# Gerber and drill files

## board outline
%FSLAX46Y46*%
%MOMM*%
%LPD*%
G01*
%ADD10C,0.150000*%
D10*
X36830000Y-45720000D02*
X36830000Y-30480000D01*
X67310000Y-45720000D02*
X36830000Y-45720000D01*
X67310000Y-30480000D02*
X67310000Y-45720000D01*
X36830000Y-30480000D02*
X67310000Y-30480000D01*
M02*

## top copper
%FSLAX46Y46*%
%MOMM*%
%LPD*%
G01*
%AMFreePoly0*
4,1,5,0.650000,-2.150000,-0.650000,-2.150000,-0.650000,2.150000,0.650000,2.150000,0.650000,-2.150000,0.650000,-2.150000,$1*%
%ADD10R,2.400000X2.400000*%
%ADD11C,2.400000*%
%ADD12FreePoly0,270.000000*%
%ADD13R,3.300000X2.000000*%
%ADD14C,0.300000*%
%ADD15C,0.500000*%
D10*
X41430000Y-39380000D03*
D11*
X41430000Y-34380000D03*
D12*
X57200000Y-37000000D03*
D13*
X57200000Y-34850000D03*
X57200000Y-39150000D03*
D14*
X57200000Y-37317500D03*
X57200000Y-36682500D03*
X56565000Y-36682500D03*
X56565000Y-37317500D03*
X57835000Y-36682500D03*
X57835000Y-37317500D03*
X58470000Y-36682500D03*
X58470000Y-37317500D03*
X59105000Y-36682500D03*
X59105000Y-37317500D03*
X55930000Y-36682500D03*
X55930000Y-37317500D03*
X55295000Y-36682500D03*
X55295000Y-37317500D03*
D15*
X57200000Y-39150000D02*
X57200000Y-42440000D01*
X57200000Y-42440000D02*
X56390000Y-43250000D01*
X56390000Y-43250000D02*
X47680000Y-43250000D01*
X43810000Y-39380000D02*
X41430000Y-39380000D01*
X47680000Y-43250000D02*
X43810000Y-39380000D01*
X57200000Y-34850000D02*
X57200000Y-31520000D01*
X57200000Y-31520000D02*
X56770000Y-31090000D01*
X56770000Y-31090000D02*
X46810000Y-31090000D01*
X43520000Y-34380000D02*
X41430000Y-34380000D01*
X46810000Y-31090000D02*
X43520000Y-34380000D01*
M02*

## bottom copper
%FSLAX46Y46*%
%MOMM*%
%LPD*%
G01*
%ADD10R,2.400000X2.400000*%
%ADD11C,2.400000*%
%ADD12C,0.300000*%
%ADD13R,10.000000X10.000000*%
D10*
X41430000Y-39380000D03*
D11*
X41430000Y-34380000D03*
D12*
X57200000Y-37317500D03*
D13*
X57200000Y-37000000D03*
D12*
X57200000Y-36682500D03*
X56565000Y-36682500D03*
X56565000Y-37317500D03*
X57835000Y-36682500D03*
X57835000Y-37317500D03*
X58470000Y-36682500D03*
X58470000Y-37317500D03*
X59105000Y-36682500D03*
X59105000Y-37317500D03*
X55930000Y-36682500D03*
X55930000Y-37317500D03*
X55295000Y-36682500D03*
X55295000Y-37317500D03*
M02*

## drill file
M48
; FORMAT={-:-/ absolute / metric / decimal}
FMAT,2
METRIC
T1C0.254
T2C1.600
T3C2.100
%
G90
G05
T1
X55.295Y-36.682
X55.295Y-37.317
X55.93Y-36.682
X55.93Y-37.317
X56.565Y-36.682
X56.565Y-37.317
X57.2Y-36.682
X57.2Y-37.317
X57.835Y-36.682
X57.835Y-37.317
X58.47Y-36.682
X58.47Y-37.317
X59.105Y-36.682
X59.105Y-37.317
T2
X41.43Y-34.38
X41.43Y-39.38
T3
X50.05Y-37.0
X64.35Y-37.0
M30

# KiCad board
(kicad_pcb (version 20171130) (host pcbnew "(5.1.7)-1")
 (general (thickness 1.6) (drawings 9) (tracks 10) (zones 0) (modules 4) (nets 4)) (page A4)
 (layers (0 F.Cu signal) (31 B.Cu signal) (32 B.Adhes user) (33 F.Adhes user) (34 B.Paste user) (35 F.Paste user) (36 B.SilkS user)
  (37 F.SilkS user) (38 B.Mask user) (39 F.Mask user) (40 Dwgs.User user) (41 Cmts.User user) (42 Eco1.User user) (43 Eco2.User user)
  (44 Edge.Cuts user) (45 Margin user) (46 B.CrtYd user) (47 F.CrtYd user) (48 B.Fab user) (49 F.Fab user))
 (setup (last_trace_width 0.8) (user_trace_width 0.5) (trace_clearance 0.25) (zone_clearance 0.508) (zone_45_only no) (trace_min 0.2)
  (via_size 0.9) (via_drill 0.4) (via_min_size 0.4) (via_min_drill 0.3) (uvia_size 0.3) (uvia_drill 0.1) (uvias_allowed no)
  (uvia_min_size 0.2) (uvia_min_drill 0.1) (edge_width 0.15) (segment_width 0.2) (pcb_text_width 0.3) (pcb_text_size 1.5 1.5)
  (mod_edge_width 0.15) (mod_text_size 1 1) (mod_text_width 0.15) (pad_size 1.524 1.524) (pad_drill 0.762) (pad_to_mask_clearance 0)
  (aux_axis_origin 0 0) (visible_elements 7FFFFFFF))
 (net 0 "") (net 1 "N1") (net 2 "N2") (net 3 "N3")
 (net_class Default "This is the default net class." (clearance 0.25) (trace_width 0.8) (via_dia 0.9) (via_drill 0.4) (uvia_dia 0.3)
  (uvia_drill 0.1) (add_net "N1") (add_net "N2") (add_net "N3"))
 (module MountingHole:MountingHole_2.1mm (layer F.Cu) (at 64.35 37)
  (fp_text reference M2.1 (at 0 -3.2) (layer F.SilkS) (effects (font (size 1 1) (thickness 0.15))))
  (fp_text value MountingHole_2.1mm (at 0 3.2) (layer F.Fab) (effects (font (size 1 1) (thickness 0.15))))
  (pad "" np_thru_hole circle (at 0 0) (size 2.1 2.1) (drill 2.1) (layers *.Cu *.Mask)))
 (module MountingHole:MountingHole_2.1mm (layer F.Cu) (at 50.05 37)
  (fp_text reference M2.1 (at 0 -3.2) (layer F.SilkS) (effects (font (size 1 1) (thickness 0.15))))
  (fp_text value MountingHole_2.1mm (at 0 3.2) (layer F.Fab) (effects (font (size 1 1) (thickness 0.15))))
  (pad "" np_thru_hole circle (at 0 0) (size 2.1 2.1) (drill 2.1) (layers *.Cu *.Mask)))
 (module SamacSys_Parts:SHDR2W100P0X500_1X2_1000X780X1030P (layer F.Cu) (at 41.43 39.38 90)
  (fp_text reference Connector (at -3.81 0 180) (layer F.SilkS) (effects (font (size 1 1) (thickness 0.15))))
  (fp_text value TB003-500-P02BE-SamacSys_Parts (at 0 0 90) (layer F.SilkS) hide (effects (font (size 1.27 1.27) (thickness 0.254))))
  (pad 1 thru_hole rect (at 0 0 90) (size 2.4 2.4) (drill 1.6) (layers *.Cu *.Mask) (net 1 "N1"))
  (pad 2 thru_hole circle (at 5 0 90) (size 2.4 2.4) (drill 1.6) (layers *.Cu *.Mask) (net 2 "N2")))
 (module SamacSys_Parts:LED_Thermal (layer F.Cu) (at 57.2 37 270)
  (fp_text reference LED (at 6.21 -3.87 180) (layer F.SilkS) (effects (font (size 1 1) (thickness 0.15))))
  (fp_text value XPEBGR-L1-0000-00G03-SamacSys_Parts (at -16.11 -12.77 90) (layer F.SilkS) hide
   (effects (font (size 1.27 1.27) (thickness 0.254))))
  (pad 3 smd custom (at 0 0 270) (size 1.3 4.3) (layers F.Cu F.Paste F.Mask) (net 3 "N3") (zone_connect 0)
   (options (clearance outline) (anchor rect)) (primitives))
  (pad 1 smd rect (at -2.15 0 270) (size 2 3.3) (layers F.Cu F.Paste F.Mask) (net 2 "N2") (zone_connect 0))
  (pad 2 smd rect (at 2.15 0 270) (size 2 3.3) (layers F.Cu F.Paste F.Mask) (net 1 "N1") (zone_connect 0))
  (pad 3 thru_hole circle (at 0.3175 0 270) (size 0.3 0.3) (drill 0.254) (layers *.Cu *.Mask) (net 3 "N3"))
  (pad 3 smd rect (at 0 0 270) (size 10 10) (layers B.Cu B.Paste B.Mask) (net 3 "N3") (zone_connect 0))
  (pad 3 thru_hole circle (at -0.3175 0 270) (size 0.3 0.3) (drill 0.254) (layers *.Cu *.Mask) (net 3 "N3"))
  (pad 3 thru_hole circle (at -0.3175 0.635 270) (size 0.3 0.3) (drill 0.254) (layers *.Cu *.Mask) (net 3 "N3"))
  (pad 3 thru_hole circle (at 0.3175 0.635 270) (size 0.3 0.3) (drill 0.254) (layers *.Cu *.Mask) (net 3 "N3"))
  (pad 3 thru_hole circle (at -0.3175 -0.635 270) (size 0.3 0.3) (drill 0.254) (layers *.Cu *.Mask) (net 3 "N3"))
  (pad 3 thru_hole circle (at 0.3175 -0.635 270) (size 0.3 0.3) (drill 0.254) (layers *.Cu *.Mask) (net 3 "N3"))
  (pad 3 thru_hole circle (at -0.3175 -1.27 270) (size 0.3 0.3) (drill 0.254) (layers *.Cu *.Mask) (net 3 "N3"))
  (pad 3 thru_hole circle (at 0.3175 -1.27 270) (size 0.3 0.3) (drill 0.254) (layers *.Cu *.Mask) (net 3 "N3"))
  (pad 3 thru_hole circle (at -0.3175 -1.905 270) (size 0.3 0.3) (drill 0.254) (layers *.Cu *.Mask) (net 3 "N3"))
  (pad 3 thru_hole circle (at 0.3175 -1.905 270) (size 0.3 0.3) (drill 0.254) (layers *.Cu *.Mask) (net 3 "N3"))
  (pad 3 thru_hole circle (at -0.3175 1.27 270) (size 0.3 0.3) (drill 0.254) (layers *.Cu *.Mask) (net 3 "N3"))
  (pad 3 thru_hole circle (at 0.3175 1.27 270) (size 0.3 0.3) (drill 0.254) (layers *.Cu *.Mask) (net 3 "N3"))
  (pad 3 thru_hole circle (at -0.3175 1.905 270) (size 0.3 0.3) (drill 0.254) (layers *.Cu *.Mask) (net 3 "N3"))
  (pad 3 thru_hole circle (at 0.3175 1.905 270) (size 0.3 0.3) (drill 0.254) (layers *.Cu *.Mask) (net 3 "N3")))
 (gr_line (start 36.83 45.72) (end 36.83 30.48) (layer Edge.Cuts) (width 0.15))
 (gr_line (start 67.31 45.72) (end 36.83 45.72) (layer Edge.Cuts) (width 0.15))
 (gr_line (start 67.31 30.48) (end 67.31 45.72) (layer Edge.Cuts) (width 0.15))
 (gr_line (start 36.83 30.48) (end 67.31 30.48) (layer Edge.Cuts) (width 0.15))
 (segment (start 57.2 39.15) (end 57.2 42.44) (width 0.5) (layer F.Cu) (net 1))
 (segment (start 57.2 42.44) (end 56.39 43.25) (width 0.5) (layer F.Cu) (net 1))
 (segment (start 56.39 43.25) (end 47.68 43.25) (width 0.5) (layer F.Cu) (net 1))
 (segment (start 43.81 39.38) (end 41.43 39.38) (width 0.5) (layer F.Cu) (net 1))
 (segment (start 47.68 43.25) (end 43.81 39.38) (width 0.5) (layer F.Cu) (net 1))
 (segment (start 57.2 34.85) (end 57.2 31.52) (width 0.5) (layer F.Cu) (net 2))
 (segment (start 57.2 31.52) (end 56.77 31.09) (width 0.5) (layer F.Cu) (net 2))
 (segment (start 56.77 31.09) (end 46.81 31.09) (width 0.5) (layer F.Cu) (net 2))
 (segment (start 43.52 34.38) (end 41.43 34.38) (width 0.5) (layer F.Cu) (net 2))
 (segment (start 46.81 31.09) (end 43.52 34.38) (width 0.5) (layer F.Cu) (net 2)))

